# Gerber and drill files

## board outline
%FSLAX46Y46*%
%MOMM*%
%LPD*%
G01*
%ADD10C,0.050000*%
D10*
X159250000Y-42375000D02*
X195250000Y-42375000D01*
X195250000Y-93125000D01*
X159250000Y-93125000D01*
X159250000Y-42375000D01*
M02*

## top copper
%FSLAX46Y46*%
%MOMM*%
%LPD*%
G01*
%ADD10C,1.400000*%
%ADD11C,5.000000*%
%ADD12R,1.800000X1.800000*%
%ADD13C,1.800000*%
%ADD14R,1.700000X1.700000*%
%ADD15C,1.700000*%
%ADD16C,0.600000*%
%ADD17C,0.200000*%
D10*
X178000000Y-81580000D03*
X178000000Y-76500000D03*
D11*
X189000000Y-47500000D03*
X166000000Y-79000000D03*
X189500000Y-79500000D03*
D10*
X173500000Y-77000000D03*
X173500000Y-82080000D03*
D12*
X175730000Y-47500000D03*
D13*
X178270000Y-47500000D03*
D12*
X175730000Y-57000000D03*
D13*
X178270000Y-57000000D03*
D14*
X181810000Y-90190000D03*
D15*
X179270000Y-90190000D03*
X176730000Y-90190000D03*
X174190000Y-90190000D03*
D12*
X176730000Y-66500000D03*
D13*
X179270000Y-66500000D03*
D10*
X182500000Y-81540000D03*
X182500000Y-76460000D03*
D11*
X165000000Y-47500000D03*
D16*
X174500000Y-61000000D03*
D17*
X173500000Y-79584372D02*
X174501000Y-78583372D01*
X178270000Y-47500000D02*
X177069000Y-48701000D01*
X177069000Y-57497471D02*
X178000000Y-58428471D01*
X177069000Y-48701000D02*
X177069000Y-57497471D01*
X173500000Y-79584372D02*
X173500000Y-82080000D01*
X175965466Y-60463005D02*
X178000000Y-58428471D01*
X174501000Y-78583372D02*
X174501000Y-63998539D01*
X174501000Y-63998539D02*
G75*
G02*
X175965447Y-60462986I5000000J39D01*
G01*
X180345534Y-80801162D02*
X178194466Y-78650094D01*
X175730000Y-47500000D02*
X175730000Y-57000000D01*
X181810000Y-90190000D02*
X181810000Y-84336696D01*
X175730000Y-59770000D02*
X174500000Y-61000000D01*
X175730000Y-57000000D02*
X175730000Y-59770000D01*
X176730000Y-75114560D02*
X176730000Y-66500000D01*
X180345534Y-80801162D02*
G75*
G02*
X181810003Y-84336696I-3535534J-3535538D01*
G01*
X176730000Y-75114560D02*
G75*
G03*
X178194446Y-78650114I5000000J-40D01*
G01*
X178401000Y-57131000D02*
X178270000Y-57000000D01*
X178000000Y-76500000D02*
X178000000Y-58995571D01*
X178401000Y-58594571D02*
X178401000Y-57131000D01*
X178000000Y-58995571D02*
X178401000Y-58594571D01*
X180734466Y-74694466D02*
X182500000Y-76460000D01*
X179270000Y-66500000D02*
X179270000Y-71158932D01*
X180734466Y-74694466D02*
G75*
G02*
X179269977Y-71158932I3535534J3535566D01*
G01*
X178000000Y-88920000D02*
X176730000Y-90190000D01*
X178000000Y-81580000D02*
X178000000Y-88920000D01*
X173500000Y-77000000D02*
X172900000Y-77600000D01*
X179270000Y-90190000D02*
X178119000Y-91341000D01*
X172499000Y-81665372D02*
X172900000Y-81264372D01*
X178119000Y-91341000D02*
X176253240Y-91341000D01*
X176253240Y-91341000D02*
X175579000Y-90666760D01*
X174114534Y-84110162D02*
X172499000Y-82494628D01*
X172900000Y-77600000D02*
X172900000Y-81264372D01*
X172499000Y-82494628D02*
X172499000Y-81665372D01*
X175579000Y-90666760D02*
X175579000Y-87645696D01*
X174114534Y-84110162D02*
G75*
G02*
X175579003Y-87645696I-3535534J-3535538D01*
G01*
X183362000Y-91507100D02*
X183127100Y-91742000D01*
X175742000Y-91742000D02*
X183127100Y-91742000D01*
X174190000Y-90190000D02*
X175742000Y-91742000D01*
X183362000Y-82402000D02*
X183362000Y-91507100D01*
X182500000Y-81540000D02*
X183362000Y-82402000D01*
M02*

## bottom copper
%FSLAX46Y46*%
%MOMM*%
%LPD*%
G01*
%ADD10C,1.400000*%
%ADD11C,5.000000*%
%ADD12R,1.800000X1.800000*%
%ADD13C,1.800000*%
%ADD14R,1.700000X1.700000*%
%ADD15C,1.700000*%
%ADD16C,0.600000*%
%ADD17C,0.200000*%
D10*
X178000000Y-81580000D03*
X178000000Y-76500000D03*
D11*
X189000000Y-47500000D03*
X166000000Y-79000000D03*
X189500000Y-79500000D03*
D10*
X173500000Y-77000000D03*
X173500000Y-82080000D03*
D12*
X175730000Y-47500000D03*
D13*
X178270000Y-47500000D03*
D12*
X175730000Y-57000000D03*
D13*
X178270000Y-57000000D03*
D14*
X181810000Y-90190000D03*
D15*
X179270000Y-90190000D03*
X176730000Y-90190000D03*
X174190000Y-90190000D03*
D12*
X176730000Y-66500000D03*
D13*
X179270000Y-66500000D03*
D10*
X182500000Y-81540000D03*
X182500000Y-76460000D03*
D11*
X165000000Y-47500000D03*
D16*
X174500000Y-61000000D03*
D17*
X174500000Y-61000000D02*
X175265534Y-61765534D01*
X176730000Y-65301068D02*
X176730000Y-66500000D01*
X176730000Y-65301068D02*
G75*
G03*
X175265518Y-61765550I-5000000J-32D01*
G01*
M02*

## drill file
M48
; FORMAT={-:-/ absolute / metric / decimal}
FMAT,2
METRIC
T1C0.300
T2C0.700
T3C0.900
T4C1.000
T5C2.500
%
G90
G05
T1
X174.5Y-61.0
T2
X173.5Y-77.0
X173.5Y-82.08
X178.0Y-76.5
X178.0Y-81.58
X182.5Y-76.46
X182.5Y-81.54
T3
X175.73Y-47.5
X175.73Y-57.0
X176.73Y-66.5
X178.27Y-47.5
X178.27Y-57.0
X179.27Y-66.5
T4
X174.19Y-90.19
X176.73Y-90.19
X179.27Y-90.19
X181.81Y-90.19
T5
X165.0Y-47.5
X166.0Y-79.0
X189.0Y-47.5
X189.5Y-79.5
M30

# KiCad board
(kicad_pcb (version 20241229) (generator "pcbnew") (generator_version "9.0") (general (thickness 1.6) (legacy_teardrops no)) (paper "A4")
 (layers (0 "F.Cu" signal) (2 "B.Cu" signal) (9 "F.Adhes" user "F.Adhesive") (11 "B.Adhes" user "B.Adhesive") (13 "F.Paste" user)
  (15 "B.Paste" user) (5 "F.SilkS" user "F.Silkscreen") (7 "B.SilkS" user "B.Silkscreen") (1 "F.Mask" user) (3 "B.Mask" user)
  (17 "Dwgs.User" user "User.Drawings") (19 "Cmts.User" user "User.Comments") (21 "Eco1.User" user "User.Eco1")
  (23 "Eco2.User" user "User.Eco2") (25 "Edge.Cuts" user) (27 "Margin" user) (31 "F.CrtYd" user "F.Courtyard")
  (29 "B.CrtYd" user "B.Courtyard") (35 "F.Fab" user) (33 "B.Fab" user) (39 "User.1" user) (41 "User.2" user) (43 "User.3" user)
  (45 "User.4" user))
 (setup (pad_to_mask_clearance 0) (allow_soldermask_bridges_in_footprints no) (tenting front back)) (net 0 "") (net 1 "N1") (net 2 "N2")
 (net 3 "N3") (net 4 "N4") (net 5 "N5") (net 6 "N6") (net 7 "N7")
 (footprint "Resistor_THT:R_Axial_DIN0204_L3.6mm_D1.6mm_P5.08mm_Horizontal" (layer "F.Cu") (at 178 81.58 90)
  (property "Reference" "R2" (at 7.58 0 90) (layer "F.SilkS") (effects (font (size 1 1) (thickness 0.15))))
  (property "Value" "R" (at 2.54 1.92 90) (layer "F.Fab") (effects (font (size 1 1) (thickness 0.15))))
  (pad "1" thru_hole circle (at 0 0 90) (size 1.4 1.4) (drill 0.7) (layers "*.Cu" "*.Mask") (remove_unused_layers no) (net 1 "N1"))
  (pad "2" thru_hole circle (at 5.08 0 90) (size 1.4 1.4) (drill 0.7) (layers "*.Cu" "*.Mask") (remove_unused_layers no) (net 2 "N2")))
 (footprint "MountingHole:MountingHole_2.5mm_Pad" (layer "F.Cu") (at 189 47.5)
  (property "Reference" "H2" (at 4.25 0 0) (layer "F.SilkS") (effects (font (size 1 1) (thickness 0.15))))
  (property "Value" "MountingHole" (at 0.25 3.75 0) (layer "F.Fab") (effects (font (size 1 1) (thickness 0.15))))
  (pad "1" thru_hole circle (at 0 0) (size 5 5) (drill 2.5) (layers "*.Cu" "*.Mask") (remove_unused_layers no) (zone_connect 2)))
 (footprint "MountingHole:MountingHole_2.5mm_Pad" (layer "F.Cu") (at 166 79)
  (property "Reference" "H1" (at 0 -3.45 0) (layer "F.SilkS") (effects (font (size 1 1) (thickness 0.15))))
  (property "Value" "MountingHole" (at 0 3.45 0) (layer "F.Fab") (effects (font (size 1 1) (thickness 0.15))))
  (pad "1" thru_hole circle (at 0 0) (size 5 5) (drill 2.5) (layers "*.Cu" "*.Mask") (remove_unused_layers no) (zone_connect 2)))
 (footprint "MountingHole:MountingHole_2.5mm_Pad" (layer "F.Cu") (at 189.5 79.5)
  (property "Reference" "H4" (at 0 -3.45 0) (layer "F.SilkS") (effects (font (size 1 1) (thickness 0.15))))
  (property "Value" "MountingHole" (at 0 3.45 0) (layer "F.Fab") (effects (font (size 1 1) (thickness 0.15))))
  (pad "1" thru_hole circle (at 0 0) (size 5 5) (drill 2.5) (layers "*.Cu" "*.Mask") (remove_unused_layers no) (zone_connect 2)))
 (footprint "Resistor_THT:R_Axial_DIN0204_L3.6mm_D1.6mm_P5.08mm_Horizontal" (layer "F.Cu") (at 173.5 77 -90)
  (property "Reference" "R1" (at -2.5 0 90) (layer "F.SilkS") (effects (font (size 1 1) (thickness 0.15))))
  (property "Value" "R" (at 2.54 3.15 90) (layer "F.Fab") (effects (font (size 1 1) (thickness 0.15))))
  (pad "1" thru_hole circle (at 0 0 270) (size 1.4 1.4) (drill 0.7) (layers "*.Cu" "*.Mask") (remove_unused_layers no) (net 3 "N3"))
  (pad "2" thru_hole circle (at 5.08 0 270) (size 1.4 1.4) (drill 0.7) (layers "*.Cu" "*.Mask") (remove_unused_layers no) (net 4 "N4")))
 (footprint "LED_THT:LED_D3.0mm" (layer "F.Cu") (at 175.73 47.5)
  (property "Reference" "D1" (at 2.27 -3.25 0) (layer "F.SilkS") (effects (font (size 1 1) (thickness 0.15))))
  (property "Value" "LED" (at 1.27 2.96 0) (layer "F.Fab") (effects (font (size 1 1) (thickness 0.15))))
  (pad "1" thru_hole rect (at 0 0) (size 1.8 1.8) (drill 0.9) (layers "*.Cu" "*.Mask") (remove_unused_layers no) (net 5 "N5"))
  (pad "2" thru_hole circle (at 2.54 0) (size 1.8 1.8) (drill 0.9) (layers "*.Cu" "*.Mask") (remove_unused_layers no) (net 4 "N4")))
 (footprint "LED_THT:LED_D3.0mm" (layer "F.Cu") (at 175.73 57)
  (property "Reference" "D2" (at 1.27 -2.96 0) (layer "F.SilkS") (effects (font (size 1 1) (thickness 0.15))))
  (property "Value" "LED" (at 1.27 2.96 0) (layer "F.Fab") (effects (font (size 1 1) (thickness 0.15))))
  (pad "1" thru_hole rect (at 0 0) (size 1.8 1.8) (drill 0.9) (layers "*.Cu" "*.Mask") (remove_unused_layers no) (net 5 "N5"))
  (pad "2" thru_hole circle (at 2.54 0) (size 1.8 1.8) (drill 0.9) (layers "*.Cu" "*.Mask") (remove_unused_layers no) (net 2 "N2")))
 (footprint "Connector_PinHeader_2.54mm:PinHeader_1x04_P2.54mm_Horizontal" (layer "F.Cu") (at 181.81 90.19 -90)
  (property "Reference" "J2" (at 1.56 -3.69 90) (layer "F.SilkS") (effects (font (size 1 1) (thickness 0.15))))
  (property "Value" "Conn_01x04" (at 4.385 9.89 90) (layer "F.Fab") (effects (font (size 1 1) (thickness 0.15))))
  (pad "1" thru_hole rect (at 0 0 270) (size 1.7 1.7) (drill 1) (layers "*.Cu" "*.Mask") (remove_unused_layers no) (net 5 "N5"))
  (pad "2" thru_hole circle (at 0 2.54 270) (size 1.7 1.7) (drill 1) (layers "*.Cu" "*.Mask") (remove_unused_layers no) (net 3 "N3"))
  (pad "3" thru_hole circle (at 0 5.08 270) (size 1.7 1.7) (drill 1) (layers "*.Cu" "*.Mask") (remove_unused_layers no) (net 1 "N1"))
  (pad "4" thru_hole circle (at 0 7.62 270) (size 1.7 1.7) (drill 1) (layers "*.Cu" "*.Mask") (remove_unused_layers no) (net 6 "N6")))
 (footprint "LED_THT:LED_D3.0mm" (layer "F.Cu") (at 176.73 66.5)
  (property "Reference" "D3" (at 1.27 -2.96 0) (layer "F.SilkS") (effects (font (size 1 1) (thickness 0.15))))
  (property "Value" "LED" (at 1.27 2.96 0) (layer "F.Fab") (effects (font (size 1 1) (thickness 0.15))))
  (pad "1" thru_hole rect (at 0 0) (size 1.8 1.8) (drill 0.9) (layers "*.Cu" "*.Mask") (remove_unused_layers no) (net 5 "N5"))
  (pad "2" thru_hole circle (at 2.54 0) (size 1.8 1.8) (drill 0.9) (layers "*.Cu" "*.Mask") (remove_unused_layers no) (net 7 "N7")))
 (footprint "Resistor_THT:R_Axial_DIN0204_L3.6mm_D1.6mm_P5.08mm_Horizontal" (layer "F.Cu") (at 182.5 81.54 90)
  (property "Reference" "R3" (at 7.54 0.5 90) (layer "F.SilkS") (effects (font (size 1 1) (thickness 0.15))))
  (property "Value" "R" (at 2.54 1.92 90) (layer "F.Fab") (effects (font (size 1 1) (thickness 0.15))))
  (pad "1" thru_hole circle (at 0 0 90) (size 1.4 1.4) (drill 0.7) (layers "*.Cu" "*.Mask") (remove_unused_layers no) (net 6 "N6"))
  (pad "2" thru_hole circle (at 5.08 0 90) (size 1.4 1.4) (drill 0.7) (layers "*.Cu" "*.Mask") (remove_unused_layers no) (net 7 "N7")))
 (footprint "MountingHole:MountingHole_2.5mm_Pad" (layer "F.Cu") (at 165 47.5)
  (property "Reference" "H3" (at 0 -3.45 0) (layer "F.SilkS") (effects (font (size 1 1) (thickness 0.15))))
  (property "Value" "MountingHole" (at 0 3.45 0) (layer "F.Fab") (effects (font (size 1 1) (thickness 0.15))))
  (pad "1" thru_hole circle (at 0 0) (size 5 5) (drill 2.5) (layers "*.Cu" "*.Mask") (remove_unused_layers no) (zone_connect 2)))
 (gr_rect (start 159.25 42.375) (end 195.25 93.125) (stroke (width 0.05) (type default)) (fill no) (layer "Edge.Cuts"))
 (segment (start 173.5 79.584372) (end 174.501 78.583372) (width 0.2) (layer "F.Cu") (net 4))
 (segment (start 178.27 47.5) (end 177.069 48.701) (width 0.2) (layer "F.Cu") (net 4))
 (segment (start 177.069 57.497471) (end 178 58.428471) (width 0.2) (layer "F.Cu") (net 4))
 (segment (start 177.069 48.701) (end 177.069 57.497471) (width 0.2) (layer "F.Cu") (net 4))
 (segment (start 173.5 79.584372) (end 173.5 82.08) (width 0.2) (layer "F.Cu") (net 4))
 (segment (start 175.965466 60.463005) (end 178 58.428471) (width 0.2) (layer "F.Cu") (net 4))
 (segment (start 174.501 78.583372) (end 174.501 63.998539) (width 0.2) (layer "F.Cu") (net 4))
 (arc (start 174.501 63.998539) (mid 174.881602 62.085122) (end 175.965466 60.463005) (width 0.2) (layer "F.Cu") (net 4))
 (segment (start 180.345534 80.801162) (end 178.194466 78.650094) (width 0.2) (layer "F.Cu") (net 5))
 (segment (start 175.73 47.5) (end 175.73 57) (width 0.2) (layer "F.Cu") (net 5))
 (segment (start 181.81 90.19) (end 181.81 84.336696) (width 0.2) (layer "F.Cu") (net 5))
 (segment (start 175.73 59.77) (end 174.5 61) (width 0.2) (layer "F.Cu") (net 5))
 (segment (start 175.73 57) (end 175.73 59.77) (width 0.2) (layer "F.Cu") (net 5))
 (segment (start 176.73 75.11456) (end 176.73 66.5) (width 0.2) (layer "F.Cu") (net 5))
 (via (at 174.5 61) (size 0.6) (drill 0.3) (layers "F.Cu" "B.Cu") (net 5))
 (arc (start 180.345534 80.801162) (mid 181.429398 82.423279) (end 181.81 84.336696) (width 0.2) (layer "F.Cu") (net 5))
 (arc (start 176.73 75.11456) (mid 177.110602 77.027977) (end 178.194466 78.650094) (width 0.2) (layer "F.Cu") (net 5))
 (segment (start 174.5 61) (end 175.265534 61.765534) (width 0.2) (layer "B.Cu") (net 5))
 (segment (start 176.73 65.301068) (end 176.73 66.5) (width 0.2) (layer "B.Cu") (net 5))
 (arc (start 176.73 65.301068) (mid 176.349398 63.387651) (end 175.265534 61.765534) (width 0.2) (layer "B.Cu") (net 5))
 (segment (start 178.401 57.131) (end 178.27 57) (width 0.2) (layer "F.Cu") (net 2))
 (segment (start 178 76.5) (end 178 58.995571) (width 0.2) (layer "F.Cu") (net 2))
 (segment (start 178.401 58.594571) (end 178.401 57.131) (width 0.2) (layer "F.Cu") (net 2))
 (segment (start 178 58.995571) (end 178.401 58.594571) (width 0.2) (layer "F.Cu") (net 2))
 (segment (start 180.734466 74.694466) (end 182.5 76.46) (width 0.2) (layer "F.Cu") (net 7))
 (segment (start 179.27 66.5) (end 179.27 71.158932) (width 0.2) (layer "F.Cu") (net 7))
 (arc (start 180.734466 74.694466) (mid 179.650602 73.072349) (end 179.27 71.158932) (width 0.2) (layer "F.Cu") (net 7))
 (segment (start 178 88.92) (end 176.73 90.19) (width 0.2) (layer "F.Cu") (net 1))
 (segment (start 178 81.58) (end 178 88.92) (width 0.2) (layer "F.Cu") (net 1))
 (segment (start 173.5 77) (end 172.9 77.6) (width 0.2) (layer "F.Cu") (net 3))
 (segment (start 179.27 90.19) (end 178.119 91.341) (width 0.2) (layer "F.Cu") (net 3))
 (segment (start 172.499 81.665372) (end 172.9 81.264372) (width 0.2) (layer "F.Cu") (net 3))
 (segment (start 178.119 91.341) (end 176.25324 91.341) (width 0.2) (layer "F.Cu") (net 3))
 (segment (start 176.25324 91.341) (end 175.579 90.66676) (width 0.2) (layer "F.Cu") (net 3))
 (segment (start 174.114534 84.110162) (end 172.499 82.494628) (width 0.2) (layer "F.Cu") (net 3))
 (segment (start 172.9 77.6) (end 172.9 81.264372) (width 0.2) (layer "F.Cu") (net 3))
 (segment (start 172.499 82.494628) (end 172.499 81.665372) (width 0.2) (layer "F.Cu") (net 3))
 (segment (start 175.579 90.66676) (end 175.579 87.645696) (width 0.2) (layer "F.Cu") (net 3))
 (arc (start 174.114534 84.110162) (mid 175.198398 85.732279) (end 175.579 87.645696) (width 0.2) (layer "F.Cu") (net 3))
 (segment (start 183.362 91.5071) (end 183.1271 91.742) (width 0.2) (layer "F.Cu") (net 6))
 (segment (start 175.742 91.742) (end 183.1271 91.742) (width 0.2) (layer "F.Cu") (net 6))
 (segment (start 174.19 90.19) (end 175.742 91.742) (width 0.2) (layer "F.Cu") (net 6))
 (segment (start 183.362 82.402) (end 183.362 91.5071) (width 0.2) (layer "F.Cu") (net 6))
 (segment (start 182.5 81.54) (end 183.362 82.402) (width 0.2) (layer "F.Cu") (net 6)))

